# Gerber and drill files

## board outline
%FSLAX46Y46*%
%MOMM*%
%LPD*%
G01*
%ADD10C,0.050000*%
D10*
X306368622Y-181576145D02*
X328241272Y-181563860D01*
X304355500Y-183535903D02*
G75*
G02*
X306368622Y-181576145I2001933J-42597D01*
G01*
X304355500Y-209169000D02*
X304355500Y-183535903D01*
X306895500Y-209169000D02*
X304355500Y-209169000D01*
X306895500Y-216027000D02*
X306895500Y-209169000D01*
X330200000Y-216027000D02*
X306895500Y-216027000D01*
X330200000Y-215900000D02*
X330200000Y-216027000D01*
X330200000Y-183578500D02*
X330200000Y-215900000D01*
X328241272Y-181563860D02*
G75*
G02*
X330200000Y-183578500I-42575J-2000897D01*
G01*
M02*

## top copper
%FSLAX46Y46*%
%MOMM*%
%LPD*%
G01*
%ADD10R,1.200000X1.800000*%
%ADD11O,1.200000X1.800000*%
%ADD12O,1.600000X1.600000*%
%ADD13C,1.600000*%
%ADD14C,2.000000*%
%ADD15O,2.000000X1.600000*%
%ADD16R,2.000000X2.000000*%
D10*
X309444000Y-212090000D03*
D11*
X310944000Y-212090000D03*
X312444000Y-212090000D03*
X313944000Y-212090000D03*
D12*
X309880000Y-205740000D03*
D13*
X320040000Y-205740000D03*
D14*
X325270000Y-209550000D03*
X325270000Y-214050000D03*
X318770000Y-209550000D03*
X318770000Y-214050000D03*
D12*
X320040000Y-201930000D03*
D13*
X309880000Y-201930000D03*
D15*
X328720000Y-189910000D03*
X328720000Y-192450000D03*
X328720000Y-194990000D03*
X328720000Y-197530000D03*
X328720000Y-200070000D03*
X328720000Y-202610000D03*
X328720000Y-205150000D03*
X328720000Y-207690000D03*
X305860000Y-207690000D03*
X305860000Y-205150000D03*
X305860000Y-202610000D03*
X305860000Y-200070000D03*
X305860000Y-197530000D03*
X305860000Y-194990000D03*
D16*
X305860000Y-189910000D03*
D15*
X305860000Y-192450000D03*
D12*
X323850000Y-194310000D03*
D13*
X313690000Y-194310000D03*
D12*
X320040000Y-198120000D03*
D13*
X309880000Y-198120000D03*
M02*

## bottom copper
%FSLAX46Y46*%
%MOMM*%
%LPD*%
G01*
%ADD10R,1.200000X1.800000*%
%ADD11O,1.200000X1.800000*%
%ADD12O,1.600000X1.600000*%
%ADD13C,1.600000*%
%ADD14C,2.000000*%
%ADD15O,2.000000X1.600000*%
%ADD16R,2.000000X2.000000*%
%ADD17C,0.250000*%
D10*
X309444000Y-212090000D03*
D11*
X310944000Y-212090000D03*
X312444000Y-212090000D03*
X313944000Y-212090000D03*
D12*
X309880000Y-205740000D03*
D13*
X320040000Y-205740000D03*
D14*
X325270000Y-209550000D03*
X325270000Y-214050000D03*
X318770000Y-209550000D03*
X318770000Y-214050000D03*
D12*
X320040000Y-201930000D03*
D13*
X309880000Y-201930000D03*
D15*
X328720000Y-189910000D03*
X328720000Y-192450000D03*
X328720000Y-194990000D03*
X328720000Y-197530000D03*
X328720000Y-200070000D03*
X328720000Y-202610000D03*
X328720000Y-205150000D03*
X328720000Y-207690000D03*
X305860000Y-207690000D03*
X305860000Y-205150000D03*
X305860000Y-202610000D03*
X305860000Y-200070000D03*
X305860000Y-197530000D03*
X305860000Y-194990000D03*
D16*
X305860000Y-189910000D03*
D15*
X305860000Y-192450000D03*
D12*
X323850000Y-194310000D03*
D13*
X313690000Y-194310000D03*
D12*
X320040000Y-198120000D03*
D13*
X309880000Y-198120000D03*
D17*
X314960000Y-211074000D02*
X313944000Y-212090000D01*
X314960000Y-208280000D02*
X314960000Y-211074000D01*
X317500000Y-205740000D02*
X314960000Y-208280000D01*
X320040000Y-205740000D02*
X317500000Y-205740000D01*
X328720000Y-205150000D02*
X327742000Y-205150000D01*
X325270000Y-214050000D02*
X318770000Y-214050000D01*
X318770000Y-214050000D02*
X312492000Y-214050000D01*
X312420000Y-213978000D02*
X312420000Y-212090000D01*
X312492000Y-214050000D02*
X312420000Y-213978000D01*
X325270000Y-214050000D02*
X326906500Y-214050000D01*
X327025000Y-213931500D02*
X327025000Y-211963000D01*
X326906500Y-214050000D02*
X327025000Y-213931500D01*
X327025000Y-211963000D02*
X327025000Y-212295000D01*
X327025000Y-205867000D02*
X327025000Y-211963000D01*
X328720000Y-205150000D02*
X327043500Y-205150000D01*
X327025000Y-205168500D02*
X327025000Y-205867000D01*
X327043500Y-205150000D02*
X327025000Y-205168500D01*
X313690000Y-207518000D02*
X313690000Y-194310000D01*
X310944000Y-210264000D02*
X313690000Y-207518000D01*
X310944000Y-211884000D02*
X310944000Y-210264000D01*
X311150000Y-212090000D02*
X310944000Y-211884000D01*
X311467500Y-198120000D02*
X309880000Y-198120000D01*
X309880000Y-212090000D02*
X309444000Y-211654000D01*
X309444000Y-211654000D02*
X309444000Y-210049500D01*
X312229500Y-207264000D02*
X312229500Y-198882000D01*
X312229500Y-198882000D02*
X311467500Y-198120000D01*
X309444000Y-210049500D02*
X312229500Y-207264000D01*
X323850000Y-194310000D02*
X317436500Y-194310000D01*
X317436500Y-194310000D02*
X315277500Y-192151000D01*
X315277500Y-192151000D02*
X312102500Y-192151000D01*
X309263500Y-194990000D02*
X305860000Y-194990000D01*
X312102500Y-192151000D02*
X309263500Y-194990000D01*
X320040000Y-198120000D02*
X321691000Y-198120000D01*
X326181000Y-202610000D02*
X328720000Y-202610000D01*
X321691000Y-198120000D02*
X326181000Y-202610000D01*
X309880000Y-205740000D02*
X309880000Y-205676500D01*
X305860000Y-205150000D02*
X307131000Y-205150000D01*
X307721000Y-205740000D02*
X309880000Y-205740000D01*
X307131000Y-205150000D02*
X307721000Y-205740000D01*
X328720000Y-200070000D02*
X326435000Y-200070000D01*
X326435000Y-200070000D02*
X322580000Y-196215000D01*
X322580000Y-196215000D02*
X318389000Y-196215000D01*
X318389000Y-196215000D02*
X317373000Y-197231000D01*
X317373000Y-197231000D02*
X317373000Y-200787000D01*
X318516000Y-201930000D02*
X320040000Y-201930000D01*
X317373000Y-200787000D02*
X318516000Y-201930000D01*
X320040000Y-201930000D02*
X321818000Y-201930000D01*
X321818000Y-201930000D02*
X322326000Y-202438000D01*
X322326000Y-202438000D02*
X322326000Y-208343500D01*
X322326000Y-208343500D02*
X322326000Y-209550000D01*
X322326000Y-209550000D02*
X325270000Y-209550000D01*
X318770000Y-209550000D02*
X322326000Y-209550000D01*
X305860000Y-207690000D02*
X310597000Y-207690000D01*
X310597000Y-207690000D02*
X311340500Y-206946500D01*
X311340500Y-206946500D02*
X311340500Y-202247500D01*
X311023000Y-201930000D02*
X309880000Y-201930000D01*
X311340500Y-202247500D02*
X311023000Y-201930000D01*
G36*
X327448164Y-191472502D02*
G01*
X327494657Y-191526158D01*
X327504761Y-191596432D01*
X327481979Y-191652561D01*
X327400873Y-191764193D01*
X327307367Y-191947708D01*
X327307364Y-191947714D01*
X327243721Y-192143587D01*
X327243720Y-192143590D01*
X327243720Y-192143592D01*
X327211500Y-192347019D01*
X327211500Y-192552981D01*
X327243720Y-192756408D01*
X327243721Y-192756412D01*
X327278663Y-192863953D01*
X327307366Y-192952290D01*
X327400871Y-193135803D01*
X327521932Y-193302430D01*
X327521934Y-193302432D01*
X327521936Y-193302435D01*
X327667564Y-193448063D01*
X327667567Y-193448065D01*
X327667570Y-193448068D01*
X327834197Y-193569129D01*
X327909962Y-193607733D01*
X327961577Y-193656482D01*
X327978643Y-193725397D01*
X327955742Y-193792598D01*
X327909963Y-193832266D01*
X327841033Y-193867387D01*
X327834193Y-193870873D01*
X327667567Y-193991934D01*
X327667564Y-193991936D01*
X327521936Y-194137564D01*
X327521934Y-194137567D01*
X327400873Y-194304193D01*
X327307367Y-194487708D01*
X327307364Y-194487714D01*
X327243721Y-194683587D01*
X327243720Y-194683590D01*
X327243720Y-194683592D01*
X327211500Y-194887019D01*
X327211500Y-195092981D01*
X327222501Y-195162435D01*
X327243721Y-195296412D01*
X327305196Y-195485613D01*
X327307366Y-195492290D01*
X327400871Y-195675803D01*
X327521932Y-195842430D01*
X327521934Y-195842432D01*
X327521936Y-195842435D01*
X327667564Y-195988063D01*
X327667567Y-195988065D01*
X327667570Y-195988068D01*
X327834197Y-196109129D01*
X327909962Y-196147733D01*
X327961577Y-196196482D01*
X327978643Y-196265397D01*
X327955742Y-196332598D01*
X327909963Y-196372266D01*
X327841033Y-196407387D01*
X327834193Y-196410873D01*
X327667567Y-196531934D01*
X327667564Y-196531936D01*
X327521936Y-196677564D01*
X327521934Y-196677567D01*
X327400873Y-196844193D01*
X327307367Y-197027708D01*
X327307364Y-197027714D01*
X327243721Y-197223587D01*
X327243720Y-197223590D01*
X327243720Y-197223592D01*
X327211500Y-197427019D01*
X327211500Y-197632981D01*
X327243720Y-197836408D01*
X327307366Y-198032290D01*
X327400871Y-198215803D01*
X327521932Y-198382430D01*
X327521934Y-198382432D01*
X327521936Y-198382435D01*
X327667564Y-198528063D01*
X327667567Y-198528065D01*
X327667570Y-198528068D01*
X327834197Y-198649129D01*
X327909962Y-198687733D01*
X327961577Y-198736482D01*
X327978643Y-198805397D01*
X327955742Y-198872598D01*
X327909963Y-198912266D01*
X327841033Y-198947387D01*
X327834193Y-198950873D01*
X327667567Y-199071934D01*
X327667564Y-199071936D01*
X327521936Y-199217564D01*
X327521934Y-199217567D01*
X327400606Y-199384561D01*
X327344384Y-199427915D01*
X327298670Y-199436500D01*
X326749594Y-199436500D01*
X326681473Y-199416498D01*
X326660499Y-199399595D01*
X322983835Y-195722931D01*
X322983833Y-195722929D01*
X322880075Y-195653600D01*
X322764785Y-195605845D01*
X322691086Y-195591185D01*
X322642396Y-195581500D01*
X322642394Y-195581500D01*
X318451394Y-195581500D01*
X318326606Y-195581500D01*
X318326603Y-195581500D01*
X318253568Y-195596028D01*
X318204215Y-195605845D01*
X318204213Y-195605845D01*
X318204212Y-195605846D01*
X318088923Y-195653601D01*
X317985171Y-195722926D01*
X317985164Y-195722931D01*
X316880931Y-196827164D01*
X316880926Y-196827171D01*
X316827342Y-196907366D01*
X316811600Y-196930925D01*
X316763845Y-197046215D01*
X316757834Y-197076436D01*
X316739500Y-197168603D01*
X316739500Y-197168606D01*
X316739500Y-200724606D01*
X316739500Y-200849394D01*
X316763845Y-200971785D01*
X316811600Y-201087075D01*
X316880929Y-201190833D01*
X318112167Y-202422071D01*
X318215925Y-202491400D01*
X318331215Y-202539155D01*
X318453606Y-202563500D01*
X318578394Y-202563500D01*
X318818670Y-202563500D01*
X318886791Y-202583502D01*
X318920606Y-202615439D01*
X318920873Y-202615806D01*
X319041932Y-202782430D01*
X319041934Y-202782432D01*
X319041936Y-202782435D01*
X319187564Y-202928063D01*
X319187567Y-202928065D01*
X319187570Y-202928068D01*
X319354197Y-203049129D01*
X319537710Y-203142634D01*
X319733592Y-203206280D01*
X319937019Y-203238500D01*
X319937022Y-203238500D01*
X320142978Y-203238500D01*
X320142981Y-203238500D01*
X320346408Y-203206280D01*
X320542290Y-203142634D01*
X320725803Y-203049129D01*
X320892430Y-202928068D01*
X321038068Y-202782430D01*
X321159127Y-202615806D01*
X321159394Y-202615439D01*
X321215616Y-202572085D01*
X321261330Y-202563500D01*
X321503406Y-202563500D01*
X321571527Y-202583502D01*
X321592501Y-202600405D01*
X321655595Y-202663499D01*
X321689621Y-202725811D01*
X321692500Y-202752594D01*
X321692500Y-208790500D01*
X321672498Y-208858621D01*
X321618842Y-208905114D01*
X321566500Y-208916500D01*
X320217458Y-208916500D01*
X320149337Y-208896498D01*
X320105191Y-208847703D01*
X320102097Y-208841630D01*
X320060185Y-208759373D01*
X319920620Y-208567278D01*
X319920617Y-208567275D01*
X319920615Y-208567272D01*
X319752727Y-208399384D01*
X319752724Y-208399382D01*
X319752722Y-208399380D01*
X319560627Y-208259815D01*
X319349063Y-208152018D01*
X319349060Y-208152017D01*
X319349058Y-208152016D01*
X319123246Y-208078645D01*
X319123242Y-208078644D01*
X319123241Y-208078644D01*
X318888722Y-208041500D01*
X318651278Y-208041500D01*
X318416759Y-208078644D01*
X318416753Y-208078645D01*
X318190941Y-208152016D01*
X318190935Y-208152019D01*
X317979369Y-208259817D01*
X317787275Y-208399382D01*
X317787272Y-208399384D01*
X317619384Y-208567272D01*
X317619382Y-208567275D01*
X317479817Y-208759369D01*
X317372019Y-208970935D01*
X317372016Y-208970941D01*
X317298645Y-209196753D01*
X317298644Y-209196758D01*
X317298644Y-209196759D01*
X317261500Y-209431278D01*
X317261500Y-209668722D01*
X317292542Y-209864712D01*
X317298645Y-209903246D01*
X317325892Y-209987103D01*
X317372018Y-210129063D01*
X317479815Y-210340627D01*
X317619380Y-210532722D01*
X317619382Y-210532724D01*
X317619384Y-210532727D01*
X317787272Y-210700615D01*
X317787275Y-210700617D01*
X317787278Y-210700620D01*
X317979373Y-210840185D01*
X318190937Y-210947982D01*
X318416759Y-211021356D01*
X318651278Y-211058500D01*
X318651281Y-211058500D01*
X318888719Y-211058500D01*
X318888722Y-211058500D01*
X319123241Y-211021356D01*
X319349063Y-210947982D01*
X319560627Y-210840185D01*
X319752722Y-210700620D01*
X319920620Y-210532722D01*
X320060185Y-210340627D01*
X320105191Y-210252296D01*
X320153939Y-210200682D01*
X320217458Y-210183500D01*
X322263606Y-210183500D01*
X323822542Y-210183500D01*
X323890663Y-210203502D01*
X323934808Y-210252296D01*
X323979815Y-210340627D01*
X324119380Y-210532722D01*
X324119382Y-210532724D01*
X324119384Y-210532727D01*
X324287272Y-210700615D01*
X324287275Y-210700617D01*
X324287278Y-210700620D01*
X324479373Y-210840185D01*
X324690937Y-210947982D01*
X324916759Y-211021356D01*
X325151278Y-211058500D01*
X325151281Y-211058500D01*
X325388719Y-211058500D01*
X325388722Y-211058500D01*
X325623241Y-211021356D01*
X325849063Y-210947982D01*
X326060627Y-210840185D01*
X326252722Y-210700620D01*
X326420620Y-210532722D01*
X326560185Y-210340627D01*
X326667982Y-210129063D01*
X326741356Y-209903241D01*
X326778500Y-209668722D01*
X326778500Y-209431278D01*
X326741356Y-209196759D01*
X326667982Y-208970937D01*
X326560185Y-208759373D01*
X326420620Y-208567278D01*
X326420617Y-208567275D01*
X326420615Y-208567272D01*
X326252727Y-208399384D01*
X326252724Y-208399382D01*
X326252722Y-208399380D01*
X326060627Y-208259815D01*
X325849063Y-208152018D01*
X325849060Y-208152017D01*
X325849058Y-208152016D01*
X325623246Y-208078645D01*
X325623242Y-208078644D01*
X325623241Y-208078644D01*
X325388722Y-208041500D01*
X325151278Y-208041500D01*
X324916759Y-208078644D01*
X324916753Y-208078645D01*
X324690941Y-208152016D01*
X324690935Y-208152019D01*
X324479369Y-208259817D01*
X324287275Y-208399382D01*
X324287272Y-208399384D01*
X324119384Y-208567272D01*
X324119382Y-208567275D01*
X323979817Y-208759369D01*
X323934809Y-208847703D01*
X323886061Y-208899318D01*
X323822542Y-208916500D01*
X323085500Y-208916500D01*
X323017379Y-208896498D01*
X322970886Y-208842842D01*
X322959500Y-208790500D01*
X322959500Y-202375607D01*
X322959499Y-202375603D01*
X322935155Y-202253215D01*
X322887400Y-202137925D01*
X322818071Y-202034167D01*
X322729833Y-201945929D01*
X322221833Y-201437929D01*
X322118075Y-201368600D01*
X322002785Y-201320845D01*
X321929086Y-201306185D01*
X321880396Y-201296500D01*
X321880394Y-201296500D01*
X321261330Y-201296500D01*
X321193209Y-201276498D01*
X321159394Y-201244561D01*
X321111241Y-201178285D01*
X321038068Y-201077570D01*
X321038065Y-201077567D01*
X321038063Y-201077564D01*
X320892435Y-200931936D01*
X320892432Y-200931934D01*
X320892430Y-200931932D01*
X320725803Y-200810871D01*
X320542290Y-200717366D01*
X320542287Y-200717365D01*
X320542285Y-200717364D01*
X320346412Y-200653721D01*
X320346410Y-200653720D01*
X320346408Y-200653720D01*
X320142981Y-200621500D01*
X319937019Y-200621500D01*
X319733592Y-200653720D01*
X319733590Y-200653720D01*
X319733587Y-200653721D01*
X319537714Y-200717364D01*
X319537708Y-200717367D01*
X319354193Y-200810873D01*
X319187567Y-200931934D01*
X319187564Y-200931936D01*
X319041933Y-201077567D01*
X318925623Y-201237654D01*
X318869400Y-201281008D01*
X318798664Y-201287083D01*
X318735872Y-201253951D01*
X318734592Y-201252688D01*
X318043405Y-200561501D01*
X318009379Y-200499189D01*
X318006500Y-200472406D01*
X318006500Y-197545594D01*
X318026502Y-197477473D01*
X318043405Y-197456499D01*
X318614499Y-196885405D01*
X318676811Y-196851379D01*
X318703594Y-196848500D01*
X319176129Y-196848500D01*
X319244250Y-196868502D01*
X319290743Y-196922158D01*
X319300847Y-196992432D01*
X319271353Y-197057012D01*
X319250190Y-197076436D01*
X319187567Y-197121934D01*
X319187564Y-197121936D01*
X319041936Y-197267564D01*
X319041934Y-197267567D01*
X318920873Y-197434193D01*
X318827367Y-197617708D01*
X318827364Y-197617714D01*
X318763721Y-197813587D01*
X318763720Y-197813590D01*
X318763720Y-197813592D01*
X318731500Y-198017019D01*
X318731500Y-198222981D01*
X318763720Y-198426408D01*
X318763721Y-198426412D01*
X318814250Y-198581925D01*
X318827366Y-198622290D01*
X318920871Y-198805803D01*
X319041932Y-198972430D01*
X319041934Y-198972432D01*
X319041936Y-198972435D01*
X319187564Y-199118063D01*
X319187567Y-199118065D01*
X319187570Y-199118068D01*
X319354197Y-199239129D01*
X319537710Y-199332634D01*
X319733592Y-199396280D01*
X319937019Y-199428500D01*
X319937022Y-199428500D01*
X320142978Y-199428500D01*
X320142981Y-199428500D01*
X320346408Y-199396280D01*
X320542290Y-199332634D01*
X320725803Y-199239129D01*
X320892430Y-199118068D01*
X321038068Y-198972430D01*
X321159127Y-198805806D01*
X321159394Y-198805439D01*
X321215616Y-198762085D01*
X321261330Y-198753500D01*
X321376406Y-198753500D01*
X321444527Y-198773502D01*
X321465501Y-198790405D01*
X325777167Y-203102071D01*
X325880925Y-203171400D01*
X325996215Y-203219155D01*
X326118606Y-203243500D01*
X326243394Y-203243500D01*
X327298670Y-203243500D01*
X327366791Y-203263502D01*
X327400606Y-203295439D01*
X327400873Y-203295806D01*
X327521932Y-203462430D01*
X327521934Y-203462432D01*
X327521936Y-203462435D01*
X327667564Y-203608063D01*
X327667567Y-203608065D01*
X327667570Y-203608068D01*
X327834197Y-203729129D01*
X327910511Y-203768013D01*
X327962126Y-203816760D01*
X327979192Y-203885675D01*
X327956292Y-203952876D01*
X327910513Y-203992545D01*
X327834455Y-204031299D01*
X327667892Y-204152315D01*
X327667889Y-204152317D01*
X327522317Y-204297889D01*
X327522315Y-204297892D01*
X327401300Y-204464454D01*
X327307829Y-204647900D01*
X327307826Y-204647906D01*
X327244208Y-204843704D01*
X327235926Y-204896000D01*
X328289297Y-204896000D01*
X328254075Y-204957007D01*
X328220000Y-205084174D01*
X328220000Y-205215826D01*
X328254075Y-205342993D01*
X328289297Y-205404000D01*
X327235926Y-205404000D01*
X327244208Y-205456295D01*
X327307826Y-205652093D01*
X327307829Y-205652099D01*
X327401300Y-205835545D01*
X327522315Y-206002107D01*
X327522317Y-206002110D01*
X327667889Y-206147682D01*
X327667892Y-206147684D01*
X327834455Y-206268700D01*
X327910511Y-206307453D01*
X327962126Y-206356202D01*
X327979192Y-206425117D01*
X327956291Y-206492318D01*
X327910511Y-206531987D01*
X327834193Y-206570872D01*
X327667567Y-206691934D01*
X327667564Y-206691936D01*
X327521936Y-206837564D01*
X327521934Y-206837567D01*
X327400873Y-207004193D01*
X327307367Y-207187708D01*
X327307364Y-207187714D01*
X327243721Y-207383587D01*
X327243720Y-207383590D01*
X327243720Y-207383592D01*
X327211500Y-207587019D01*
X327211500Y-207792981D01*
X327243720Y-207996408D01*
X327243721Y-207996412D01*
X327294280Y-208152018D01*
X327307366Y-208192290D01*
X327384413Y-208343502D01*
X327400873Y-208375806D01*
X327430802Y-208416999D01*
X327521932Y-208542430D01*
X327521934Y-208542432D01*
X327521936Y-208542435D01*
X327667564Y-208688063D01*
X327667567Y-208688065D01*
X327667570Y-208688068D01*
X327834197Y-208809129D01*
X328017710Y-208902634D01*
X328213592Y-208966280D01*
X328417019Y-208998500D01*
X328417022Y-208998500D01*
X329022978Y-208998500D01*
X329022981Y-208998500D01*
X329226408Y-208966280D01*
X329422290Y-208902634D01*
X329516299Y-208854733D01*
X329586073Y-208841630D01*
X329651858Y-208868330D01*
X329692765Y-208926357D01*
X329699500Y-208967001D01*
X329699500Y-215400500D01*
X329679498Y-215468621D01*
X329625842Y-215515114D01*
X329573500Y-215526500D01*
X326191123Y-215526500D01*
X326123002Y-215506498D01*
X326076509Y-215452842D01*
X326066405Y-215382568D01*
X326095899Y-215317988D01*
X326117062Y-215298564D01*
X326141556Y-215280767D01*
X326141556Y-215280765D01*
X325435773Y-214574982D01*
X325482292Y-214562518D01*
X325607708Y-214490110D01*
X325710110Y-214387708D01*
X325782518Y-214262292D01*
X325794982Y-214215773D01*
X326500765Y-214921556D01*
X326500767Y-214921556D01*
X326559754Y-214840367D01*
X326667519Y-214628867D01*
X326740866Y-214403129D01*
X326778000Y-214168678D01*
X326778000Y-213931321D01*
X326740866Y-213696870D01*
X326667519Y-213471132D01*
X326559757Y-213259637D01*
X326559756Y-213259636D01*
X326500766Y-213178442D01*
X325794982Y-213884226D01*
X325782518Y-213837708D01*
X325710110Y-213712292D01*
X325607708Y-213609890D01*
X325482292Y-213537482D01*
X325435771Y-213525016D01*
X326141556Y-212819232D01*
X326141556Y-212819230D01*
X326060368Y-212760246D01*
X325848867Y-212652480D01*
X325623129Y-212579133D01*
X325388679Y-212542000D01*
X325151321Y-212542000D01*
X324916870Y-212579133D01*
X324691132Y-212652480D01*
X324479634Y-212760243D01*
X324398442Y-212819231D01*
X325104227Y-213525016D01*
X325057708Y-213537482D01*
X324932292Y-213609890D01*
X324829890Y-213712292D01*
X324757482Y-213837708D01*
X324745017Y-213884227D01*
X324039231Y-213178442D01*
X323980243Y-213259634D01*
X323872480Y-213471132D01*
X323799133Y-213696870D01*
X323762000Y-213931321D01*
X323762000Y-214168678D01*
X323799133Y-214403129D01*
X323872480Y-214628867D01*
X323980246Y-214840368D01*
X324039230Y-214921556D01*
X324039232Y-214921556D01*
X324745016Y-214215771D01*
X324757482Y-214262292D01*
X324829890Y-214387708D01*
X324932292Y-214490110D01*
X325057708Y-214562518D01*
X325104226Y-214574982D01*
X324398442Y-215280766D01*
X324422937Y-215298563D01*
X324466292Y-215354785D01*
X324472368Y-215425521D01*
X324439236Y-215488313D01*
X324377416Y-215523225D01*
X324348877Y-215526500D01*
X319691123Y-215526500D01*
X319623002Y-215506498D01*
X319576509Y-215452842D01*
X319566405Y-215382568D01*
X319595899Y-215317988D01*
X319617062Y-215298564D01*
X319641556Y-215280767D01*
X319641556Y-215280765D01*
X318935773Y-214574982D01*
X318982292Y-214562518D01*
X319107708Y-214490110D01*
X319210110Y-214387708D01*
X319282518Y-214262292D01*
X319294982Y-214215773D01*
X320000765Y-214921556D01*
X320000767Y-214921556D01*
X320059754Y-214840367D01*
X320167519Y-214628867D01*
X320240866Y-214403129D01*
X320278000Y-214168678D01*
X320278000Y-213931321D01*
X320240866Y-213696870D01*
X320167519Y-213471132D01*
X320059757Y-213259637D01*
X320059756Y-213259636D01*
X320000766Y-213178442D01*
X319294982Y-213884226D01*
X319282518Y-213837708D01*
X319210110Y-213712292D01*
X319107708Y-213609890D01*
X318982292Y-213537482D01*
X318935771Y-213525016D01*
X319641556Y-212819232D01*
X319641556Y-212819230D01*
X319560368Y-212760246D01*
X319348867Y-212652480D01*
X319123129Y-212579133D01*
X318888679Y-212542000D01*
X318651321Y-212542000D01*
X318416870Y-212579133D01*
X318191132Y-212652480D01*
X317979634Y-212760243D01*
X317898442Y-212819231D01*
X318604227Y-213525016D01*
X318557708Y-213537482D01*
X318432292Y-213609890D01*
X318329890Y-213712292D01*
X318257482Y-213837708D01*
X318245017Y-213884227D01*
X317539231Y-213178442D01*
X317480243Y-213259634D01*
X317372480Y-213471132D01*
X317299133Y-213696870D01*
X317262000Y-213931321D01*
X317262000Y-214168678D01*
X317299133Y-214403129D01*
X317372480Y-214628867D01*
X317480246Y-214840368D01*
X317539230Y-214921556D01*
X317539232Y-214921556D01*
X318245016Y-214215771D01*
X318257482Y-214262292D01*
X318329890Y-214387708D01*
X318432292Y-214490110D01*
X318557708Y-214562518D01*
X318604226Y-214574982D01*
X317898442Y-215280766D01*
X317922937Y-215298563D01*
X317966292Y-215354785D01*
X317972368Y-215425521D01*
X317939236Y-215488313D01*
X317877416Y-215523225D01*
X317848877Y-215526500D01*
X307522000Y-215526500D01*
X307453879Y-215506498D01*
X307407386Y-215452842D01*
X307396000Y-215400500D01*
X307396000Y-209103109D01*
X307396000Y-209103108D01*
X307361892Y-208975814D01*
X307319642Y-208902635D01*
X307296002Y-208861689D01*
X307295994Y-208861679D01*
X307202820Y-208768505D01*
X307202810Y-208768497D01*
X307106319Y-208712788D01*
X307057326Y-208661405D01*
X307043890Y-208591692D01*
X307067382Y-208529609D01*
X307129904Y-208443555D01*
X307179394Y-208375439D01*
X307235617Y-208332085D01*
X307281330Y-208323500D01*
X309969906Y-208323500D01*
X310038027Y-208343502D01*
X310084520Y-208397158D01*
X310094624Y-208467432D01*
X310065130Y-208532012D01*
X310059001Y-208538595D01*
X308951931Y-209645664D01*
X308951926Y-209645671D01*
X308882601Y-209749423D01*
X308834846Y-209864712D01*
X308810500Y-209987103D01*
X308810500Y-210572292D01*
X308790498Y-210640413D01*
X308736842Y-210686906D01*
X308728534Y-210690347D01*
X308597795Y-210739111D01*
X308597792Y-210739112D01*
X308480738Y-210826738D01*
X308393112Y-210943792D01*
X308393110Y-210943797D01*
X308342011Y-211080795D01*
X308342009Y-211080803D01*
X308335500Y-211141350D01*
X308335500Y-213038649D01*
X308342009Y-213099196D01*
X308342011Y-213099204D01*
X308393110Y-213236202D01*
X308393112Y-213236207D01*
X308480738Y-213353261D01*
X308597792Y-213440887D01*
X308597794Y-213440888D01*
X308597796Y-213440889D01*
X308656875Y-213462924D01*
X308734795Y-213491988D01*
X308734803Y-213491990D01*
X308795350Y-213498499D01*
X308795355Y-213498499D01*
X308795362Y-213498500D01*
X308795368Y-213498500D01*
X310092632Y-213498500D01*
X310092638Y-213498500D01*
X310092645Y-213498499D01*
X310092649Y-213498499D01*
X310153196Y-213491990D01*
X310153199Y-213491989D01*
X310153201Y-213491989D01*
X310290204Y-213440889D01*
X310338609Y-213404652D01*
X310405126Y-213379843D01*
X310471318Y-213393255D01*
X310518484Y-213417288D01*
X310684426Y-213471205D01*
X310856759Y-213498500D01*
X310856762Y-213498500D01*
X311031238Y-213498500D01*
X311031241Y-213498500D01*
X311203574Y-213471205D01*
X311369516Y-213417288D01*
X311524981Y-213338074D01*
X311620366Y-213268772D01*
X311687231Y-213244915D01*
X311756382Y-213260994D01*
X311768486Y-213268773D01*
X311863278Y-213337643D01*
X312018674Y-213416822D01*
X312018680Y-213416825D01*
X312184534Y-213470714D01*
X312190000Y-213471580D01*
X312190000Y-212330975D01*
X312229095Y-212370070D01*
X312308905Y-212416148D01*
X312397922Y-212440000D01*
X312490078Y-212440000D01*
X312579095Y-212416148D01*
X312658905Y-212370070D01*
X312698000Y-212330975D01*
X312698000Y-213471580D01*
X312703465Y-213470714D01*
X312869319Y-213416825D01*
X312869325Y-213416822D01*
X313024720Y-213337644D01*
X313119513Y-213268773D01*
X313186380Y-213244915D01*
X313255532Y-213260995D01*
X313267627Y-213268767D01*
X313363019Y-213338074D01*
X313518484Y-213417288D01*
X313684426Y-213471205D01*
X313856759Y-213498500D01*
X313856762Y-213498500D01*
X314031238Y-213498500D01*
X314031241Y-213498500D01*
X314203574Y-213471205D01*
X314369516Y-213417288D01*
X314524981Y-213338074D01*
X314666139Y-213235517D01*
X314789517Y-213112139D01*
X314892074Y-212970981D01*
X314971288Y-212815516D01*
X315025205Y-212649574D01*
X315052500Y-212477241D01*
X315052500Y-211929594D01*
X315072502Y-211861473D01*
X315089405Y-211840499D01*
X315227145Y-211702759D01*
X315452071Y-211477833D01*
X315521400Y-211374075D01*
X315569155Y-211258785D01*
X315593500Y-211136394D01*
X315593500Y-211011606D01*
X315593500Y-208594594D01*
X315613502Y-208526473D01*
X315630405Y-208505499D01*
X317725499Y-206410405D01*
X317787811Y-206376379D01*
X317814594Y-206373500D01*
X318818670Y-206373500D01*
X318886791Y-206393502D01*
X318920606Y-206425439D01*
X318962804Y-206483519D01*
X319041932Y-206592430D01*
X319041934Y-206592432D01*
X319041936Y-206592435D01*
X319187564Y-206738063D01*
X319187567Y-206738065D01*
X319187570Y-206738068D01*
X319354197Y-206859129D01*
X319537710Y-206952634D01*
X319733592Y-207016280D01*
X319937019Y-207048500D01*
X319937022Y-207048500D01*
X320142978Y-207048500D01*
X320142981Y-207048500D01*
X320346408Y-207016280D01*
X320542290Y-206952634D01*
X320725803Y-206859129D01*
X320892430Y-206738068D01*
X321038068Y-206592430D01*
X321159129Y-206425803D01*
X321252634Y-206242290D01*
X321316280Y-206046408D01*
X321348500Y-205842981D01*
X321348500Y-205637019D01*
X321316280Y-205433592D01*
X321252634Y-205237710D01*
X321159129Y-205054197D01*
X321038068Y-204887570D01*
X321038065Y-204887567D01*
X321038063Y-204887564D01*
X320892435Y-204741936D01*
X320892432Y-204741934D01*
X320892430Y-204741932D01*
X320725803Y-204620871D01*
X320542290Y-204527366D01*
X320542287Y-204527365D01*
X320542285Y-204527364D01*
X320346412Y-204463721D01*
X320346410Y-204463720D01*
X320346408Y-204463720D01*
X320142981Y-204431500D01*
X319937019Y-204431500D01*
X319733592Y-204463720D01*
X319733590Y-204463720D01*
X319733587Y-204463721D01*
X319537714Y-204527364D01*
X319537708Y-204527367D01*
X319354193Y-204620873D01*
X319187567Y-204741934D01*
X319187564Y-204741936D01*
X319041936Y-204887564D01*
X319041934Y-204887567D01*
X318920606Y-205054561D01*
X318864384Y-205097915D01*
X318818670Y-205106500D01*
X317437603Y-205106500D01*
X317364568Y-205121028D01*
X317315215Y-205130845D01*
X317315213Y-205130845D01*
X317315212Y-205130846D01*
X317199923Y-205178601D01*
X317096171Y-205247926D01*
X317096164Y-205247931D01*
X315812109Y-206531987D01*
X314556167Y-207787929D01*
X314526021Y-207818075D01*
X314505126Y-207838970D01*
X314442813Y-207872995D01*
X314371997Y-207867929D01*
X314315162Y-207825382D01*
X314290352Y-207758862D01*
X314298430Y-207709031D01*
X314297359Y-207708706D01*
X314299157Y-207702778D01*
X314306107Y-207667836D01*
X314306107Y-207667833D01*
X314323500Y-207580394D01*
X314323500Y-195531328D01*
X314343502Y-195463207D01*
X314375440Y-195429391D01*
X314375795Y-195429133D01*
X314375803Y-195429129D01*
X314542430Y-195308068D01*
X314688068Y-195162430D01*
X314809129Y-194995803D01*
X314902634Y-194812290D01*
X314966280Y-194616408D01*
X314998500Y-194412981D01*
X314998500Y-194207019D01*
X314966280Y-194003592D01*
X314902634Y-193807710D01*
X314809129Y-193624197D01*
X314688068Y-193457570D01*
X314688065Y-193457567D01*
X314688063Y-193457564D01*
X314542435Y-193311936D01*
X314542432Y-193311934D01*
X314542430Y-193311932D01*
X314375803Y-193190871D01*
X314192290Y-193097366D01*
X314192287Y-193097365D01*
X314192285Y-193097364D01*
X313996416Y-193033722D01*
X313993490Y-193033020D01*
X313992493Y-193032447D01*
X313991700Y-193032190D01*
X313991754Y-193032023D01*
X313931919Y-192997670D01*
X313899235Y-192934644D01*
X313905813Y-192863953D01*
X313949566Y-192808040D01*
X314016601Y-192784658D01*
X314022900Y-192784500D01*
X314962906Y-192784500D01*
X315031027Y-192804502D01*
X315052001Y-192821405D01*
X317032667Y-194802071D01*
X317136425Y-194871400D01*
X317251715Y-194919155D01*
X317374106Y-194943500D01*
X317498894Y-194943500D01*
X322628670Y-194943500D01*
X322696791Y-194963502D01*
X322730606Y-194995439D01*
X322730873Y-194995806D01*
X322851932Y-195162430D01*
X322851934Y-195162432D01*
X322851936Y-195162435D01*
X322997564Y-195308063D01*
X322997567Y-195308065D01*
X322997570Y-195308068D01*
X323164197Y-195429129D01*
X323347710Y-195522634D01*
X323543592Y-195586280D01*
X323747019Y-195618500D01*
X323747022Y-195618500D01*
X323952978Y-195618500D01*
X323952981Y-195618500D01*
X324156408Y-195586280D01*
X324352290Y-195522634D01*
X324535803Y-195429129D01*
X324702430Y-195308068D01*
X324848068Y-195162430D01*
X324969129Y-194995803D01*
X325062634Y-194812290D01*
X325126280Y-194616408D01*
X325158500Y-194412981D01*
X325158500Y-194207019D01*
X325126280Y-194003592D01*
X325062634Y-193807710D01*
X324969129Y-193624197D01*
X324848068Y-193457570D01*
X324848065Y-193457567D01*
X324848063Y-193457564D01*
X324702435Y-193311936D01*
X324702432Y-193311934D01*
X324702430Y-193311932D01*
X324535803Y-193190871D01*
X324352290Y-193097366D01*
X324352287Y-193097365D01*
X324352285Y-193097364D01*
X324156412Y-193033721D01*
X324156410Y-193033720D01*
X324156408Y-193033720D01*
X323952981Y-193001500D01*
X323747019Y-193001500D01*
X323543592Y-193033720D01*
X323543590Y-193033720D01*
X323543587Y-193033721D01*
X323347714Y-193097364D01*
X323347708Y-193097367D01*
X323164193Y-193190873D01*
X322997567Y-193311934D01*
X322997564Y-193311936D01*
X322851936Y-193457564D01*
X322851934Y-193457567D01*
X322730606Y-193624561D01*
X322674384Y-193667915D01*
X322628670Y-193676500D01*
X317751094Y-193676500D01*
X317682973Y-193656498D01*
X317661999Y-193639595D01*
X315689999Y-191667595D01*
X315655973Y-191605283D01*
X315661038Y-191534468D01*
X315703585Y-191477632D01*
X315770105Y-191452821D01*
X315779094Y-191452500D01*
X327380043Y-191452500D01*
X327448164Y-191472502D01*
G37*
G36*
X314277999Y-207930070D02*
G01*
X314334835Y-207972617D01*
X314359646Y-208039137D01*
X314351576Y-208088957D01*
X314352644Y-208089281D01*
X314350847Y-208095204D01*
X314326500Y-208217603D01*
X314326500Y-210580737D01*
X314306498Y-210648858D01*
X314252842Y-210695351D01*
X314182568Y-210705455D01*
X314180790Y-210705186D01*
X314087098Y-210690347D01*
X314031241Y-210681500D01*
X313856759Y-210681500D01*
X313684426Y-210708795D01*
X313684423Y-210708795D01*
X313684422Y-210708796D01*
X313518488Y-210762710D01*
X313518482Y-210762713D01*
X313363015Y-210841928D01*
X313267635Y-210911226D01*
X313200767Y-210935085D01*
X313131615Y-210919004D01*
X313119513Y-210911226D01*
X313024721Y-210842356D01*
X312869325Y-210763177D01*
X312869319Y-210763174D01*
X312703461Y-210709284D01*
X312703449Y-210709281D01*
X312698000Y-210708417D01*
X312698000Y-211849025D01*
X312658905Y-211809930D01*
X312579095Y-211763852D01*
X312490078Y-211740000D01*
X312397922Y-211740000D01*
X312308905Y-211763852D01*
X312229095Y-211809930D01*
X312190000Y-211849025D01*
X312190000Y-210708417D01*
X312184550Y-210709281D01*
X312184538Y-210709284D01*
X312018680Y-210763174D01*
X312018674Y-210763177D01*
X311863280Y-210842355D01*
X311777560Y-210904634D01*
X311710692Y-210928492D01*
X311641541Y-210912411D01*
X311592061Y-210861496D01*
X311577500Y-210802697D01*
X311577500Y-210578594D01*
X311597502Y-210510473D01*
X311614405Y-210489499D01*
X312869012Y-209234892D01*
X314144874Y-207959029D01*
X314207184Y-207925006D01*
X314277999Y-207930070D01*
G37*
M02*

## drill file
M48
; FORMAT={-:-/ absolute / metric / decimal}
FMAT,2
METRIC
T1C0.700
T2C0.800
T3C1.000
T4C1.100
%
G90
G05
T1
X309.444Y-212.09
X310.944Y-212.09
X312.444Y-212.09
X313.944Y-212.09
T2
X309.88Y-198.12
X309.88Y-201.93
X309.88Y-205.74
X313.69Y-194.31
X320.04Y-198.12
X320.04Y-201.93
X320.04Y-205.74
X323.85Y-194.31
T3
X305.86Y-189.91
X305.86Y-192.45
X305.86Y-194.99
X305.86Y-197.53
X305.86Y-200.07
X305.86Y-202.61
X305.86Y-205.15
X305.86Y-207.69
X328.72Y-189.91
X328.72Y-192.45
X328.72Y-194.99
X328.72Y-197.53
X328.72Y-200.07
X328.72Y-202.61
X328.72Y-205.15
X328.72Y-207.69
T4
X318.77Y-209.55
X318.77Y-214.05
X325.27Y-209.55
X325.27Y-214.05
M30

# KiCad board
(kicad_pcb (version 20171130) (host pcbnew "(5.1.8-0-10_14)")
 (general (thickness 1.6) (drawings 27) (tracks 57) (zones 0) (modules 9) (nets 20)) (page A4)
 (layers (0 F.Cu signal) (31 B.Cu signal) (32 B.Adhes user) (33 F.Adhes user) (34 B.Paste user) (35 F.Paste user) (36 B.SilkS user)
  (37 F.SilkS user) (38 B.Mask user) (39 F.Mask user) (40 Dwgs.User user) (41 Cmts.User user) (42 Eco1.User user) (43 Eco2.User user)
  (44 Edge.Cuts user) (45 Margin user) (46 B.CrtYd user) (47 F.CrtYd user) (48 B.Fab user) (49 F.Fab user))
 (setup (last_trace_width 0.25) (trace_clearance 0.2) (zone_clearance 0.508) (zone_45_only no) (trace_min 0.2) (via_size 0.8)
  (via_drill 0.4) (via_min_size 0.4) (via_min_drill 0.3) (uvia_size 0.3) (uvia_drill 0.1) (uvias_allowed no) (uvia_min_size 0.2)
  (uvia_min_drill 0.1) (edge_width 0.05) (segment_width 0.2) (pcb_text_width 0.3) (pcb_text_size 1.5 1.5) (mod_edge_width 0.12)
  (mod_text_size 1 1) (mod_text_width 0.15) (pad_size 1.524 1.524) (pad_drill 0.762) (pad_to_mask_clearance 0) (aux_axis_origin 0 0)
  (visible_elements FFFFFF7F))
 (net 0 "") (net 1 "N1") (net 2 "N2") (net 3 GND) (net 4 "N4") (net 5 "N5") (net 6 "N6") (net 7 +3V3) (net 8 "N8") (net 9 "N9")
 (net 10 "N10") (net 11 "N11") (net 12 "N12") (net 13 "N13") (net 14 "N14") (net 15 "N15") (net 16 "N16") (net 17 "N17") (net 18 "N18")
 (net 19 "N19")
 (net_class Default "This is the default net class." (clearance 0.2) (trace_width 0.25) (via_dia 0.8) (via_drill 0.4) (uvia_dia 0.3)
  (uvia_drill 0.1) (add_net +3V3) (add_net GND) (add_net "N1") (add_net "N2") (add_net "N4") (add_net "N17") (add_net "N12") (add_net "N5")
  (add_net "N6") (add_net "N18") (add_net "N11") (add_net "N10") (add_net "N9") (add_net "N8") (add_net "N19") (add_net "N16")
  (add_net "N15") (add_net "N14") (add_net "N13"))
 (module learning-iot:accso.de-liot (layer B.Cu) (at 317.5 187.706)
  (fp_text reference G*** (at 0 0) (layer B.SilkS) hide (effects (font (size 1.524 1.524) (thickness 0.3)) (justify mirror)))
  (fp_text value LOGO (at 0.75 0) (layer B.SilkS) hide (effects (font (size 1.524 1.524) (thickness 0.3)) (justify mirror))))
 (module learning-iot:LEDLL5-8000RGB (layer F.Cu) (at 313.69 212.09 180)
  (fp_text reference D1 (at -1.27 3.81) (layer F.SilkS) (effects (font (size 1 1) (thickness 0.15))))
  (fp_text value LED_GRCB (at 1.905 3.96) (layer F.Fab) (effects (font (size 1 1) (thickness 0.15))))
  (pad 1 thru_hole rect (at 4.246 0) (size 1.2 1.8) (drill 0.7) (layers *.Cu *.Mask) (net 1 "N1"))
  (pad 2 thru_hole oval (at 2.746 0) (size 1.2 1.8) (drill 0.7) (layers *.Cu *.Mask) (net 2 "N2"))
  (pad 3 thru_hole oval (at 1.246 0) (size 1.2 1.8) (drill 0.7) (layers *.Cu *.Mask) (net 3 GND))
  (pad 4 thru_hole oval (at -0.254 0) (size 1.2 1.8) (drill 0.7) (layers *.Cu *.Mask) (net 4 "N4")))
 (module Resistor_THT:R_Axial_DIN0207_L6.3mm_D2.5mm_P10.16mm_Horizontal (layer F.Cu) (at 320.04 205.74 180)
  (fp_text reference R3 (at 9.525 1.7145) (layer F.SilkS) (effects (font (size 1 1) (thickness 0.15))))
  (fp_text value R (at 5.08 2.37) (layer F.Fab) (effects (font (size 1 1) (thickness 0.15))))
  (pad 2 thru_hole oval (at 10.16 0 180) (size 1.6 1.6) (drill 0.8) (layers *.Cu *.Mask) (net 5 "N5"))
  (pad 1 thru_hole circle (at 0 0 180) (size 1.6 1.6) (drill 0.8) (layers *.Cu *.Mask) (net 4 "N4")))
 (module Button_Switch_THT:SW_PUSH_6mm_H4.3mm (layer F.Cu) (at 318.77 209.55)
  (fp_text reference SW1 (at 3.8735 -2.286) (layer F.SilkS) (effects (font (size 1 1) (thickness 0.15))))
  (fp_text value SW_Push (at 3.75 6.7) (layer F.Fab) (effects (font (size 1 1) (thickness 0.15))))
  (pad 1 thru_hole circle (at 6.5 0 90) (size 2 2) (drill 1.1) (layers *.Cu *.Mask) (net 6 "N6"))
  (pad 2 thru_hole circle (at 6.5 4.5 90) (size 2 2) (drill 1.1) (layers *.Cu *.Mask) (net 3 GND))
  (pad 1 thru_hole circle (at 0 0 90) (size 2 2) (drill 1.1) (layers *.Cu *.Mask) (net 6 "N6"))
  (pad 2 thru_hole circle (at 0 4.5 90) (size 2 2) (drill 1.1) (layers *.Cu *.Mask) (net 3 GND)))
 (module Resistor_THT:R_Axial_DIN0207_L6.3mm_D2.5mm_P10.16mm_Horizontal (layer F.Cu) (at 309.88 201.93)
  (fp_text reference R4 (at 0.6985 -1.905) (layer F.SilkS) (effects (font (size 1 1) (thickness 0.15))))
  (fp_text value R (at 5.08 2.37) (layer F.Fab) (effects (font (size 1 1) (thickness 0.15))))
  (pad 2 thru_hole oval (at 10.16 0) (size 1.6 1.6) (drill 0.8) (layers *.Cu *.Mask) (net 6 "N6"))
  (pad 1 thru_hole circle (at 0 0) (size 1.6 1.6) (drill 0.8) (layers *.Cu *.Mask) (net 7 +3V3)))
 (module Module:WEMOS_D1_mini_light (layer F.Cu) (at 305.86 189.91)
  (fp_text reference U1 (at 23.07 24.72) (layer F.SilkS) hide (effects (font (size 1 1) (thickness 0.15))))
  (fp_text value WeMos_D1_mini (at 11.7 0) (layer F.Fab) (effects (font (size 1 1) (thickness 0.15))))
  (pad 16 thru_hole oval (at 22.86 0) (size 2 1.6) (drill 1) (layers *.Cu *.Mask) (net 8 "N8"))
  (pad 15 thru_hole oval (at 22.86 2.54) (size 2 1.6) (drill 1) (layers *.Cu *.Mask) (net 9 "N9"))
  (pad 14 thru_hole oval (at 22.86 5.08) (size 2 1.6) (drill 1) (layers *.Cu *.Mask) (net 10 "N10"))
  (pad 13 thru_hole oval (at 22.86 7.62) (size 2 1.6) (drill 1) (layers *.Cu *.Mask) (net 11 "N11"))
  (pad 12 thru_hole oval (at 22.86 10.16) (size 2 1.6) (drill 1) (layers *.Cu *.Mask) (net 6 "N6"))
  (pad 11 thru_hole oval (at 22.86 12.7) (size 2 1.6) (drill 1) (layers *.Cu *.Mask) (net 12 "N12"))
  (pad 10 thru_hole oval (at 22.86 15.24) (size 2 1.6) (drill 1) (layers *.Cu *.Mask) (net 3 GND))
  (pad 9 thru_hole oval (at 22.86 17.78) (size 2 1.6) (drill 1) (layers *.Cu *.Mask) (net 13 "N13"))
  (pad 8 thru_hole oval (at 0 17.78) (size 2 1.6) (drill 1) (layers *.Cu *.Mask) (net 7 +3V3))
  (pad 7 thru_hole oval (at 0 15.24) (size 2 1.6) (drill 1) (layers *.Cu *.Mask) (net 5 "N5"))
  (pad 6 thru_hole oval (at 0 12.7) (size 2 1.6) (drill 1) (layers *.Cu *.Mask) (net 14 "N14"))
  (pad 5 thru_hole oval (at 0 10.16) (size 2 1.6) (drill 1) (layers *.Cu *.Mask) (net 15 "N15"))
  (pad 4 thru_hole oval (at 0 7.62) (size 2 1.6) (drill 1) (layers *.Cu *.Mask) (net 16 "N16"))
  (pad 3 thru_hole oval (at 0 5.08) (size 2 1.6) (drill 1) (layers *.Cu *.Mask) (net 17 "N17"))
  (pad 1 thru_hole rect (at 0 0) (size 2 2) (drill 1) (layers *.Cu *.Mask) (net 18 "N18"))
  (pad 2 thru_hole oval (at 0 2.54) (size 2 1.6) (drill 1) (layers *.Cu *.Mask) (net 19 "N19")))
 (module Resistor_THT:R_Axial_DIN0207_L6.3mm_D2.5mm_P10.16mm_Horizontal (layer F.Cu) (at 313.69 194.31)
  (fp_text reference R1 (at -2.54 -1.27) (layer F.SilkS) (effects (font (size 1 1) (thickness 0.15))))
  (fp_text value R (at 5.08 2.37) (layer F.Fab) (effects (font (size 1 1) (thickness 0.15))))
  (pad 2 thru_hole oval (at 10.16 0) (size 1.6 1.6) (drill 0.8) (layers *.Cu *.Mask) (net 17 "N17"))
  (pad 1 thru_hole circle (at 0 0) (size 1.6 1.6) (drill 0.8) (layers *.Cu *.Mask) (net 2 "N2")))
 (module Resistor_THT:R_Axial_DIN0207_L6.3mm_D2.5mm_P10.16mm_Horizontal (layer F.Cu) (at 309.88 198.12)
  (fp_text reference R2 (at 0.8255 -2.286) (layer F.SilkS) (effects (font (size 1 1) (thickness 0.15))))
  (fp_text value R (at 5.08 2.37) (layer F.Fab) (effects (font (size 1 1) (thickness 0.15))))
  (pad 2 thru_hole oval (at 10.16 0) (size 1.6 1.6) (drill 0.8) (layers *.Cu *.Mask) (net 12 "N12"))
  (pad 1 thru_hole circle (at 0 0) (size 1.6 1.6) (drill 0.8) (layers *.Cu *.Mask) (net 1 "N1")))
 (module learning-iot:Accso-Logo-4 (layer F.Cu) (at 318.008 185.547)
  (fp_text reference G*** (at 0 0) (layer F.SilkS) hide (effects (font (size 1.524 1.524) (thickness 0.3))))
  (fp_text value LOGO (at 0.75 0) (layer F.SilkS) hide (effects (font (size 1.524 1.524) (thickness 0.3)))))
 (gr_line (start 306.368622 181.576145) (end 328.241272 181.56386) (layer Edge.Cuts) (width 0.05))
 (gr_arc (start 306.357433 183.5785) (end 306.368622 181.576145) (angle -89.10121716) (layer Edge.Cuts) (width 0.05))
 (gr_line (start 304.3555 209.169) (end 304.3555 183.535903) (layer Edge.Cuts) (width 0.05))
 (gr_line (start 306.8955 209.169) (end 304.3555 209.169) (layer Edge.Cuts) (width 0.05))
 (gr_line (start 306.8955 216.027) (end 306.8955 209.169) (layer Edge.Cuts) (width 0.05))
 (gr_line (start 330.2 216.027) (end 306.8955 216.027) (layer Edge.Cuts) (width 0.05))
 (gr_line (start 330.2 215.9) (end 330.2 216.027) (layer Edge.Cuts) (width 0.05))
 (gr_line (start 330.2 183.5785) (end 330.2 215.9) (layer Edge.Cuts) (width 0.05))
 (gr_arc (start 328.198697 183.564757) (end 330.2 183.5785) (angle -89.17449862) (layer Edge.Cuts) (width 0.05))
 (segment (start 314.96 211.074) (end 313.944 212.09) (width 0.25) (layer B.Cu) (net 4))
 (segment (start 314.96 208.28) (end 314.96 211.074) (width 0.25) (layer B.Cu) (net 4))
 (segment (start 317.5 205.74) (end 314.96 208.28) (width 0.25) (layer B.Cu) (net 4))
 (segment (start 320.04 205.74) (end 317.5 205.74) (width 0.25) (layer B.Cu) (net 4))
 (segment (start 328.72 205.15) (end 327.742 205.15) (width 0.25) (layer B.Cu) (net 3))
 (segment (start 325.27 214.05) (end 318.77 214.05) (width 0.25) (layer B.Cu) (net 3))
 (segment (start 318.77 214.05) (end 312.492 214.05) (width 0.25) (layer B.Cu) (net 3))
 (segment (start 312.42 213.978) (end 312.42 212.09) (width 0.25) (layer B.Cu) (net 3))
 (segment (start 312.492 214.05) (end 312.42 213.978) (width 0.25) (layer B.Cu) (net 3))
 (segment (start 325.27 214.05) (end 326.9065 214.05) (width 0.25) (layer B.Cu) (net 3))
 (segment (start 327.025 213.9315) (end 327.025 211.963) (width 0.25) (layer B.Cu) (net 3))
 (segment (start 326.9065 214.05) (end 327.025 213.9315) (width 0.25) (layer B.Cu) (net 3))
 (segment (start 327.025 211.963) (end 327.025 212.295) (width 0.25) (layer B.Cu) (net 3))
 (segment (start 327.025 205.867) (end 327.025 211.963) (width 0.25) (layer B.Cu) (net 3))
 (segment (start 328.72 205.15) (end 327.0435 205.15) (width 0.25) (layer B.Cu) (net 3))
 (segment (start 327.025 205.1685) (end 327.025 205.867) (width 0.25) (layer B.Cu) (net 3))
 (segment (start 327.0435 205.15) (end 327.025 205.1685) (width 0.25) (layer B.Cu) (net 3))
 (segment (start 313.69 207.518) (end 313.69 194.31) (width 0.25) (layer B.Cu) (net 2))
 (segment (start 310.944 210.264) (end 313.69 207.518) (width 0.25) (layer B.Cu) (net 2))
 (segment (start 310.944 211.884) (end 310.944 210.264) (width 0.25) (layer B.Cu) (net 2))
 (segment (start 311.15 212.09) (end 310.944 211.884) (width 0.25) (layer B.Cu) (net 2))
 (segment (start 311.4675 198.12) (end 309.88 198.12) (width 0.25) (layer B.Cu) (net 1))
 (segment (start 309.88 212.09) (end 309.444 211.654) (width 0.25) (layer B.Cu) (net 1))
 (segment (start 309.444 211.654) (end 309.444 210.0495) (width 0.25) (layer B.Cu) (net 1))
 (segment (start 312.2295 207.264) (end 312.2295 198.882) (width 0.25) (layer B.Cu) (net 1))
 (segment (start 312.2295 198.882) (end 311.4675 198.12) (width 0.25) (layer B.Cu) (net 1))
 (segment (start 309.444 210.0495) (end 312.2295 207.264) (width 0.25) (layer B.Cu) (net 1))
 (segment (start 323.85 194.31) (end 317.4365 194.31) (width 0.25) (layer B.Cu) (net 17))
 (segment (start 317.4365 194.31) (end 315.2775 192.151) (width 0.25) (layer B.Cu) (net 17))
 (segment (start 315.2775 192.151) (end 312.1025 192.151) (width 0.25) (layer B.Cu) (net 17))
 (segment (start 309.2635 194.99) (end 305.86 194.99) (width 0.25) (layer B.Cu) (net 17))
 (segment (start 312.1025 192.151) (end 309.2635 194.99) (width 0.25) (layer B.Cu) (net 17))
 (segment (start 320.04 198.12) (end 321.691 198.12) (width 0.25) (layer B.Cu) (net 12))
 (segment (start 326.181 202.61) (end 328.72 202.61) (width 0.25) (layer B.Cu) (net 12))
 (segment (start 321.691 198.12) (end 326.181 202.61) (width 0.25) (layer B.Cu) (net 12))
 (segment (start 309.88 205.74) (end 309.88 205.6765) (width 0.25) (layer B.Cu) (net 5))
 (segment (start 305.86 205.15) (end 307.131 205.15) (width 0.25) (layer B.Cu) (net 5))
 (segment (start 307.721 205.74) (end 309.88 205.74) (width 0.25) (layer B.Cu) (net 5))
 (segment (start 307.131 205.15) (end 307.721 205.74) (width 0.25) (layer B.Cu) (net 5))
 (segment (start 328.72 200.07) (end 326.435 200.07) (width 0.25) (layer B.Cu) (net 6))
 (segment (start 326.435 200.07) (end 322.58 196.215) (width 0.25) (layer B.Cu) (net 6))
 (segment (start 322.58 196.215) (end 318.389 196.215) (width 0.25) (layer B.Cu) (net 6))
 (segment (start 318.389 196.215) (end 317.373 197.231) (width 0.25) (layer B.Cu) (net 6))
 (segment (start 317.373 197.231) (end 317.373 200.787) (width 0.25) (layer B.Cu) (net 6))
 (segment (start 318.516 201.93) (end 320.04 201.93) (width 0.25) (layer B.Cu) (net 6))
 (segment (start 317.373 200.787) (end 318.516 201.93) (width 0.25) (layer B.Cu) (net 6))
 (segment (start 320.04 201.93) (end 321.818 201.93) (width 0.25) (layer B.Cu) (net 6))
 (segment (start 321.818 201.93) (end 322.326 202.438) (width 0.25) (layer B.Cu) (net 6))
 (segment (start 322.326 202.438) (end 322.326 208.3435) (width 0.25) (layer B.Cu) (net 6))
 (segment (start 322.326 208.3435) (end 322.326 209.55) (width 0.25) (layer B.Cu) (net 6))
 (segment (start 322.326 209.55) (end 325.27 209.55) (width 0.25) (layer B.Cu) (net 6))
 (segment (start 318.77 209.55) (end 322.326 209.55) (width 0.25) (layer B.Cu) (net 6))
 (segment (start 305.86 207.69) (end 310.597 207.69) (width 0.25) (layer B.Cu) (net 7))
 (segment (start 310.597 207.69) (end 311.3405 206.9465) (width 0.25) (layer B.Cu) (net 7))
 (segment (start 311.3405 206.9465) (end 311.3405 202.2475) (width 0.25) (layer B.Cu) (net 7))
 (segment (start 311.023 201.93) (end 309.88 201.93) (width 0.25) (layer B.Cu) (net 7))
 (segment (start 311.3405 202.2475) (end 311.023 201.93) (width 0.25) (layer B.Cu) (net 7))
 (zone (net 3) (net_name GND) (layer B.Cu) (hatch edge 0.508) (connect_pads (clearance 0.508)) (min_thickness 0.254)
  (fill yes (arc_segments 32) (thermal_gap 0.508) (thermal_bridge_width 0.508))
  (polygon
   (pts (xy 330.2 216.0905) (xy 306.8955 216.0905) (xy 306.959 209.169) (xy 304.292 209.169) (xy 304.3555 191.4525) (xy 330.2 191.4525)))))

